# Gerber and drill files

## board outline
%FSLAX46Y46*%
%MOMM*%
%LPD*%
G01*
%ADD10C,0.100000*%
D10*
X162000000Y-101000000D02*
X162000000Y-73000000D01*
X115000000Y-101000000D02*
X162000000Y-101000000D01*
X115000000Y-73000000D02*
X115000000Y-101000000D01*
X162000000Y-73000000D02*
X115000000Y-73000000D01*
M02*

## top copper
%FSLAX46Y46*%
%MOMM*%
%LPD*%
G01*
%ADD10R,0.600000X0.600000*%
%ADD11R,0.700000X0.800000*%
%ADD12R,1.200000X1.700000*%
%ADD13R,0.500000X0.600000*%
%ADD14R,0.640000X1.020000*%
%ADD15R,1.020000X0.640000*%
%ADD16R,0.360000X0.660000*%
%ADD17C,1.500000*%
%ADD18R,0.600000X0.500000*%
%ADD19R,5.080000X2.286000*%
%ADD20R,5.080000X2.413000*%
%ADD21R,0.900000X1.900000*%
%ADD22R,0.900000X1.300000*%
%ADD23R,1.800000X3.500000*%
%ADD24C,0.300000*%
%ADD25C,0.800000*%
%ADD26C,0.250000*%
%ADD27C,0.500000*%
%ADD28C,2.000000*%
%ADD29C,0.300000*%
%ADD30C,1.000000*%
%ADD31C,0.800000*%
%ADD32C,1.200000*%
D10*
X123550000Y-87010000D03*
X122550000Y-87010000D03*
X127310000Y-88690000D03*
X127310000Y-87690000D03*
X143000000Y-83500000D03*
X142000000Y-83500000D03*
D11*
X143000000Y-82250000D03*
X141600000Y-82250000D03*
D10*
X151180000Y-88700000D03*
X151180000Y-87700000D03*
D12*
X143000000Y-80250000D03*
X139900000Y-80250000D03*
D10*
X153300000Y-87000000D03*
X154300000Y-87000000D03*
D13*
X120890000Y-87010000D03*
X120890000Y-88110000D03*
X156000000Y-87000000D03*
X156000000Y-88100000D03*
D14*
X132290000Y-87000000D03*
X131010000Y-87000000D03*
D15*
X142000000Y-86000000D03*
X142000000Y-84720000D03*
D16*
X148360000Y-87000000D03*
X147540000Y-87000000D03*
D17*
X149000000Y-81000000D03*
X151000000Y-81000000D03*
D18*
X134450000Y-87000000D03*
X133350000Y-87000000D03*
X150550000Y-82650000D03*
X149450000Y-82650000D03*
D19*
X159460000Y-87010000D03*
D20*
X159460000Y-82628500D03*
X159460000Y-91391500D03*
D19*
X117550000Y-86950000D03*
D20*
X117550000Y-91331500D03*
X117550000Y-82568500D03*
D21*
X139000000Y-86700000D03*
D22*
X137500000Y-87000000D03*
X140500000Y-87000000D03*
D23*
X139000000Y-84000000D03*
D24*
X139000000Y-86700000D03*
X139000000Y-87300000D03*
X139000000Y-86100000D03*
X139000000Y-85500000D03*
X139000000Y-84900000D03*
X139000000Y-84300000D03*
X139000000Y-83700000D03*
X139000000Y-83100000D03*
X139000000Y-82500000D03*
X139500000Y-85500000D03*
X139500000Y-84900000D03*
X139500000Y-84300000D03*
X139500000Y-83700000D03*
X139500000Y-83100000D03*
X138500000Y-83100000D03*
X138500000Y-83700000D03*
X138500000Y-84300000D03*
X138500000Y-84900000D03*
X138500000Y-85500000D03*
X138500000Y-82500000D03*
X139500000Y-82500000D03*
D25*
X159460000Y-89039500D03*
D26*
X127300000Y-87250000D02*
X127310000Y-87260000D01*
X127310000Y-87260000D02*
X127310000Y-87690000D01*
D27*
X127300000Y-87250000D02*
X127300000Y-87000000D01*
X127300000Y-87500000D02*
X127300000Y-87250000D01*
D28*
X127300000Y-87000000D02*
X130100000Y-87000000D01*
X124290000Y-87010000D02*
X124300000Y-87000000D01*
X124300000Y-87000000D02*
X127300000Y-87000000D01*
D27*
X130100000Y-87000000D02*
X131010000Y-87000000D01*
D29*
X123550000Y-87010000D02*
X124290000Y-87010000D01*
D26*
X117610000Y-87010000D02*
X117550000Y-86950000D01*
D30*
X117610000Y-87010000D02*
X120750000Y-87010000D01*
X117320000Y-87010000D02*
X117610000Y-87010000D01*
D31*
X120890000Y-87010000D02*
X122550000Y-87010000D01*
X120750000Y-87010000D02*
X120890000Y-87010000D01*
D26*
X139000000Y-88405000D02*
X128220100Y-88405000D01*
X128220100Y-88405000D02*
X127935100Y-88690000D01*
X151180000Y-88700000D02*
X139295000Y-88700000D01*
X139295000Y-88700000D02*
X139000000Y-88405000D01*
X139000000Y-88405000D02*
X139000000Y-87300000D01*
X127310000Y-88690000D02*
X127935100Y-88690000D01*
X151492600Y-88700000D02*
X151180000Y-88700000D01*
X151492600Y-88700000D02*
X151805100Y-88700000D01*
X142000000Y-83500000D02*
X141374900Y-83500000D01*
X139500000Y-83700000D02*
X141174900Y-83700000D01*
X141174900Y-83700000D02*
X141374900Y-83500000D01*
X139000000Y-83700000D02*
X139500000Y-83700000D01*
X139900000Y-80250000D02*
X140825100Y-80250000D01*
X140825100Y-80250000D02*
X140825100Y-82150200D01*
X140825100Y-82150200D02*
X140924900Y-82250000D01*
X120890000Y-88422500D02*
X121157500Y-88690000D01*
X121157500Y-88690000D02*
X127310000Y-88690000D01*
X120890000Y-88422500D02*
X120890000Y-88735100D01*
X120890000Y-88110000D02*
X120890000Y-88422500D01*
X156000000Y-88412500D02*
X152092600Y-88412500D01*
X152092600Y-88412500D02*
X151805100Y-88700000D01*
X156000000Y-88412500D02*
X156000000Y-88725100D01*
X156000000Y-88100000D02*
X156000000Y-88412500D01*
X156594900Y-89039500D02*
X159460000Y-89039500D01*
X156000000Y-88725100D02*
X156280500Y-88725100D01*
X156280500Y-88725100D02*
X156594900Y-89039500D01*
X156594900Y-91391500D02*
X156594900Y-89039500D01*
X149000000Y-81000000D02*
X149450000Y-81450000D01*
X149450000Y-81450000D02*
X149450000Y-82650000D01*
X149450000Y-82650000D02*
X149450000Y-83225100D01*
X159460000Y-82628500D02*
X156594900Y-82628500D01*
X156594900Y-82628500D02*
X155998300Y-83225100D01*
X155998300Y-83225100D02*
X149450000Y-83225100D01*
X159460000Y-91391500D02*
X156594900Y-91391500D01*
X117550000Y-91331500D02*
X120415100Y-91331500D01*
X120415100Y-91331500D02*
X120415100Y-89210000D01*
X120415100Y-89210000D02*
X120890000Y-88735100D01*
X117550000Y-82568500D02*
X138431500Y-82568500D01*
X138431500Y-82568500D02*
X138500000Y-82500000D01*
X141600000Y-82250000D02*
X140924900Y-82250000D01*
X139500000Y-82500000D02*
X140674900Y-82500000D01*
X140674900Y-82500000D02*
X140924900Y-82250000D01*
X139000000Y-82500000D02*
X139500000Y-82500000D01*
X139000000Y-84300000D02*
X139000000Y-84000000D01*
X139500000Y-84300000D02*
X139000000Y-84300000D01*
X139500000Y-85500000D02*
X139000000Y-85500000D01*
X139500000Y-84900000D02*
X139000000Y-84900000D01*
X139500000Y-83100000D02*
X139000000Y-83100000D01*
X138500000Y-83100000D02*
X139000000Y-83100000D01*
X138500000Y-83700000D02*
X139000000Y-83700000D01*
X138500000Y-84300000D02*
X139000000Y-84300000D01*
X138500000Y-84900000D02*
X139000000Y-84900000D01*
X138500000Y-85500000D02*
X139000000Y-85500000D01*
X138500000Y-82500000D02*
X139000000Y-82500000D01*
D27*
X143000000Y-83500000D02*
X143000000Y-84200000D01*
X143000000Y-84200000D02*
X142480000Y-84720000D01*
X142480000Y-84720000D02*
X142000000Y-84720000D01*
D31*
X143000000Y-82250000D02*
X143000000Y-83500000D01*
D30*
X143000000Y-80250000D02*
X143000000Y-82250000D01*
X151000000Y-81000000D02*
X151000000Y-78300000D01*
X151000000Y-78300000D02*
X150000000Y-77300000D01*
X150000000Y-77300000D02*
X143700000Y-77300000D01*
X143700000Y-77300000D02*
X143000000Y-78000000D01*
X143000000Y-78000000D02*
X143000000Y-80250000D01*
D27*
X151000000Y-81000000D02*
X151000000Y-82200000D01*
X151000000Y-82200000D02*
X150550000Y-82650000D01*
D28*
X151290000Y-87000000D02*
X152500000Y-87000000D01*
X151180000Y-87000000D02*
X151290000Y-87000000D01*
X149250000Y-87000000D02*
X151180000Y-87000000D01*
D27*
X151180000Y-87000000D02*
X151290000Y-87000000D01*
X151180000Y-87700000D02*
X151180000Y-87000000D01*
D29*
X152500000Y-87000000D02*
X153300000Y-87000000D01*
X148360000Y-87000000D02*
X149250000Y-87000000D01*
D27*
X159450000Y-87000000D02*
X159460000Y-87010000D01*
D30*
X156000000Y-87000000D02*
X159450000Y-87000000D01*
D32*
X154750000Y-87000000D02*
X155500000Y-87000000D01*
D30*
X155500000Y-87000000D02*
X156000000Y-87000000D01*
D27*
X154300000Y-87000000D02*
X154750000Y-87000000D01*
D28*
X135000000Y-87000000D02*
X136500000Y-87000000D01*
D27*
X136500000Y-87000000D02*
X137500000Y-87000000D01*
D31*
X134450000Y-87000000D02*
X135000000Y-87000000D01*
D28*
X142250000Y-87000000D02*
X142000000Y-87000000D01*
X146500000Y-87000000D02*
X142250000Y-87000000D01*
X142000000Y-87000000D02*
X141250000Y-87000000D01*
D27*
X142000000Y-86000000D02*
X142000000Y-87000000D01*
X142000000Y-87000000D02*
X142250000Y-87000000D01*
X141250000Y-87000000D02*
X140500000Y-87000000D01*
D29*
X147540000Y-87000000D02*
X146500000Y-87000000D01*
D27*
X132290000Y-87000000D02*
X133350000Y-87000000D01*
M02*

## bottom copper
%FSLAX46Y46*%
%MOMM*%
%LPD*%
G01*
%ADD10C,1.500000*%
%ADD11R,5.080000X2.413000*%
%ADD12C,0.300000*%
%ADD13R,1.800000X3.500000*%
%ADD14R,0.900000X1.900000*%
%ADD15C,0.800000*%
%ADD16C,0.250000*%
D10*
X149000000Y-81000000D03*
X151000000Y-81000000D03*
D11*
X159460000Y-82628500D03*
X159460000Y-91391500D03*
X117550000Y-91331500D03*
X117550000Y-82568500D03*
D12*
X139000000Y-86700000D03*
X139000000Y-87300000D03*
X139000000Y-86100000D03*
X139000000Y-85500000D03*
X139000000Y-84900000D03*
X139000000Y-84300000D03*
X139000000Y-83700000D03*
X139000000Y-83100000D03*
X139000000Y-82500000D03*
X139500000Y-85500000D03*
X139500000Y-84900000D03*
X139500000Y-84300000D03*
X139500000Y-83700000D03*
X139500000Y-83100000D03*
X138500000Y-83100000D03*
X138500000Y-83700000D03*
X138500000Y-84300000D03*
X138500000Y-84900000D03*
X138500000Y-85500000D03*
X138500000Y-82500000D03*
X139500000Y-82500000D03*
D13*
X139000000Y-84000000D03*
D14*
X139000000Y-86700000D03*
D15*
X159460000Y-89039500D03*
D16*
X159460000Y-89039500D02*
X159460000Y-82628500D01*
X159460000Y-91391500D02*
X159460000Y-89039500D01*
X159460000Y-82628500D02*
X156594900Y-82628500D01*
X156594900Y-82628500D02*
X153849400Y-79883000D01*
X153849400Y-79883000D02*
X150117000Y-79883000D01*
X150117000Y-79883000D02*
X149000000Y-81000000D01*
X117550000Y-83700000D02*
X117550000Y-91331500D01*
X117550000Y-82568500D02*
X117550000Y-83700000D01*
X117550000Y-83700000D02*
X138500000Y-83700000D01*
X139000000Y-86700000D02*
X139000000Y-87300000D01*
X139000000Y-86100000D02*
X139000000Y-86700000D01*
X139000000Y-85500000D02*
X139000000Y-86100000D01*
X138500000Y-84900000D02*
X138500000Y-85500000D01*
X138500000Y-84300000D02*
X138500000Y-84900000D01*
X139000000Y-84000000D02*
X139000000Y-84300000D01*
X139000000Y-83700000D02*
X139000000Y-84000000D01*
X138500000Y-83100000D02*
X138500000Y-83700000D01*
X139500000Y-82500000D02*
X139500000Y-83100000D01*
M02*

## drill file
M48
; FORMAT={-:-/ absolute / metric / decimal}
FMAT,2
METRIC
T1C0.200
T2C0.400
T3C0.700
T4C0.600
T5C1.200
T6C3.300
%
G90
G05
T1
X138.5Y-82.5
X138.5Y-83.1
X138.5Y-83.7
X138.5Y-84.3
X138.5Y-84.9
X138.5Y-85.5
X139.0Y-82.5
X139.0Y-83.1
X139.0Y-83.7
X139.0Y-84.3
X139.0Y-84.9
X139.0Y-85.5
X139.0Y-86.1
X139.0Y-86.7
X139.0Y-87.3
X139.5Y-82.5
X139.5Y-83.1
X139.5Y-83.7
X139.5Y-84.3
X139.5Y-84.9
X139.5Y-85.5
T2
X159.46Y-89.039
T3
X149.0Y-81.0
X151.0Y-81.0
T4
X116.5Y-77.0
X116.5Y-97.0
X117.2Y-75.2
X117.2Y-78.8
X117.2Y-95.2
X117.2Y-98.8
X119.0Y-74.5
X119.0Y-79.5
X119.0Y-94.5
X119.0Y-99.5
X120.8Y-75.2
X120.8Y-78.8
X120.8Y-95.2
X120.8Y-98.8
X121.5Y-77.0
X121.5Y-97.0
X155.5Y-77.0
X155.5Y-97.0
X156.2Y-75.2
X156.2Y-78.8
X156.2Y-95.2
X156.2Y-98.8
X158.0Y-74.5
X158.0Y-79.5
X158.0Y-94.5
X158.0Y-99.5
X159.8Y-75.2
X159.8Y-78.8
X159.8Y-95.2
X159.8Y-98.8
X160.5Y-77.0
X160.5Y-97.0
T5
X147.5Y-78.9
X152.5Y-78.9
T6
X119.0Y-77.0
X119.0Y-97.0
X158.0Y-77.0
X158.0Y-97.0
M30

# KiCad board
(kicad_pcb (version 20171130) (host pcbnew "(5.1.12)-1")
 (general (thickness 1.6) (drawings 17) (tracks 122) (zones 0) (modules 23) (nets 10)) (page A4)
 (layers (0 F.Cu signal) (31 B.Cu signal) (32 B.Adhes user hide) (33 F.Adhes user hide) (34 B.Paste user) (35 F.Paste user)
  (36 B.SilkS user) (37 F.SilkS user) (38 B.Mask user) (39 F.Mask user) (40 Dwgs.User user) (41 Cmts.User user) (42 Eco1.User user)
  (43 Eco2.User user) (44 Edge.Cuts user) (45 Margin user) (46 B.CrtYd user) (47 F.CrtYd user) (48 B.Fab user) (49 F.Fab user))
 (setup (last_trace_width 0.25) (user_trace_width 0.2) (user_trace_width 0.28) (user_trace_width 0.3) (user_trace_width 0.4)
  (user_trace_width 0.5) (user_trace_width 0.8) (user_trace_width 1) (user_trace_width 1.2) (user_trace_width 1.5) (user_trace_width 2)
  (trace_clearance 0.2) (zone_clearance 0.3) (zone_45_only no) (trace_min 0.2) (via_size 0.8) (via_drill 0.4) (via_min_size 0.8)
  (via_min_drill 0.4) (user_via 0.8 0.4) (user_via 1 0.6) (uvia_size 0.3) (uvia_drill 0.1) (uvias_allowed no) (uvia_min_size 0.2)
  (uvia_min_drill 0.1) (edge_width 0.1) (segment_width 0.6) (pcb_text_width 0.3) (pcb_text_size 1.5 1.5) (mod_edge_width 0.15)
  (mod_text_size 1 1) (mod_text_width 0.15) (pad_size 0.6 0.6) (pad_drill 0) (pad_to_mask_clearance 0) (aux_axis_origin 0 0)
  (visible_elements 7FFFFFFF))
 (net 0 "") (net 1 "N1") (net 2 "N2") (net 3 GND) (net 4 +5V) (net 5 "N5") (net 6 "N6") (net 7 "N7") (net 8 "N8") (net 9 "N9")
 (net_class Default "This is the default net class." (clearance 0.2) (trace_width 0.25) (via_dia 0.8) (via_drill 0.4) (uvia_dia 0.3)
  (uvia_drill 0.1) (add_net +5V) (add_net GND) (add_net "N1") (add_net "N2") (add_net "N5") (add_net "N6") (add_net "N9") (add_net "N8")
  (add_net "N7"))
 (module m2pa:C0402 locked (layer F.Cu) (at 123.55 87.01 180)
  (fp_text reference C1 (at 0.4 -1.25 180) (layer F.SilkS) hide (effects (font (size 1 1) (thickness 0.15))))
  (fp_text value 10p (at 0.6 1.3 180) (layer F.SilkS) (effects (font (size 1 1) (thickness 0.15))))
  (pad 1 smd rect (at 0 0 180) (size 0.6 0.6) (layers F.Cu F.Paste F.Mask) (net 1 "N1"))
  (pad 2 smd rect (at 1 0 180) (size 0.6 0.6) (layers F.Cu F.Paste F.Mask) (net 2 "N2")))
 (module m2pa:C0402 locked (layer F.Cu) (at 127.31 88.69 90)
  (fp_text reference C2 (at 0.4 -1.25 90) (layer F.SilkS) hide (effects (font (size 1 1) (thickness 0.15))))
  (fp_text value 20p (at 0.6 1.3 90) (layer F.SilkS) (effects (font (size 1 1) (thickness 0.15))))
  (pad 1 smd rect (at 0 0 90) (size 0.6 0.6) (layers F.Cu F.Paste F.Mask) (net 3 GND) (zone_connect 2))
  (pad 2 smd rect (at 1 0 90) (size 0.6 0.6) (layers F.Cu F.Paste F.Mask) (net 1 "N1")))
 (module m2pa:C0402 (layer F.Cu) (at 143 83.5 180)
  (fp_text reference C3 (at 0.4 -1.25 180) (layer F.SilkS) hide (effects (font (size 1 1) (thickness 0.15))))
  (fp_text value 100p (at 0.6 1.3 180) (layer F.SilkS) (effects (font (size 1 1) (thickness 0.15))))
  (pad 1 smd rect (at 0 0 180) (size 0.6 0.6) (layers F.Cu F.Paste F.Mask) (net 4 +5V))
  (pad 2 smd rect (at 1 0 180) (size 0.6 0.6) (layers F.Cu F.Paste F.Mask) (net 3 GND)))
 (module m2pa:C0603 (layer F.Cu) (at 143 82.25 180)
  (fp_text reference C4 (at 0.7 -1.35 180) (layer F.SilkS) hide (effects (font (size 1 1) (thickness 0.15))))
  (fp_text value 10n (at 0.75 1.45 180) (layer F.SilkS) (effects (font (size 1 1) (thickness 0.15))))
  (pad 1 smd rect (at 0 0 180) (size 0.7 0.8) (layers F.Cu F.Paste F.Mask) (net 4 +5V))
  (pad 2 smd rect (at 1.4 0 180) (size 0.7 0.8) (layers F.Cu F.Paste F.Mask) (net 3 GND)))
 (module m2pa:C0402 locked (layer F.Cu) (at 151.18 88.7 90)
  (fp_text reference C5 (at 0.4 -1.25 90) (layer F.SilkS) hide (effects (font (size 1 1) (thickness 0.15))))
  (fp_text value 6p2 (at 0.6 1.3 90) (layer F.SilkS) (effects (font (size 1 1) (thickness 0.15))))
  (pad 1 smd rect (at 0 0 90) (size 0.6 0.6) (layers F.Cu F.Paste F.Mask) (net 3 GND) (zone_connect 2))
  (pad 2 smd rect (at 1 0 90) (size 0.6 0.6) (layers F.Cu F.Paste F.Mask) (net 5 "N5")))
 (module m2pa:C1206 (layer F.Cu) (at 143 80.25 180)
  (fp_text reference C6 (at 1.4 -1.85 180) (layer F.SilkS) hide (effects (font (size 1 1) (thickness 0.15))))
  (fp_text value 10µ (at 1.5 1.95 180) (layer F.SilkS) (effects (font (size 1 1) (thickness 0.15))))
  (pad 1 smd rect (at 0 0 180) (size 1.2 1.7) (layers F.Cu F.Paste F.Mask) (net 4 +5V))
  (pad 2 smd rect (at 3.1 0 180) (size 1.2 1.7) (layers F.Cu F.Paste F.Mask) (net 3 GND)))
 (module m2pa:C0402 (layer F.Cu) (at 153.3 87)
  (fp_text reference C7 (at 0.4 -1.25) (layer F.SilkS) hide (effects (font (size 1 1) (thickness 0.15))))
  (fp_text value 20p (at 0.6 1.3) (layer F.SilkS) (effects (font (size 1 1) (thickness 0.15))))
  (pad 1 smd rect (at 0 0) (size 0.6 0.6) (layers F.Cu F.Paste F.Mask) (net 5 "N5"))
  (pad 2 smd rect (at 1 0) (size 0.6 0.6) (layers F.Cu F.Paste F.Mask) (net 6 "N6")))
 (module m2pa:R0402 (layer F.Cu) (at 120.89 87.01 270)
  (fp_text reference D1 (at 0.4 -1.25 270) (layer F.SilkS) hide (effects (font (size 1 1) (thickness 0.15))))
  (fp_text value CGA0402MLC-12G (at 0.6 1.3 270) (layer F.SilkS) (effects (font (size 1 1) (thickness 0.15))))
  (pad 1 smd rect (at 0 0 270) (size 0.6 0.5) (layers F.Cu F.Paste F.Mask) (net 2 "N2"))
  (pad 2 smd rect (at 1.1 0 270) (size 0.6 0.5) (layers F.Cu F.Paste F.Mask) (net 3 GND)))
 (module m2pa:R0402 (layer F.Cu) (at 156 87 270)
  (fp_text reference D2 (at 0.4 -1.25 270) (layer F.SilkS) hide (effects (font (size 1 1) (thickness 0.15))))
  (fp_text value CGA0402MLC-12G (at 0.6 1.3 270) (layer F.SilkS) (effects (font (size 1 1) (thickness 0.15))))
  (pad 1 smd rect (at 0 0 270) (size 0.6 0.5) (layers F.Cu F.Paste F.Mask) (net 6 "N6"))
  (pad 2 smd rect (at 1.1 0 270) (size 0.6 0.5) (layers F.Cu F.Paste F.Mask) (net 3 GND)))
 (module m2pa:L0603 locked (layer F.Cu) (at 132.29 87 180)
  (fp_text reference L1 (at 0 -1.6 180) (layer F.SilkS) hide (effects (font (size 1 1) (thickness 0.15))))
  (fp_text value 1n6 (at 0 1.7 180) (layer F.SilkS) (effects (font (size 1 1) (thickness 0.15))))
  (pad 1 smd rect (at 0 0 180) (size 0.64 1.02) (layers F.Cu F.Paste F.Mask) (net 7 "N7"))
  (pad 2 smd rect (at 1.28 0 180) (size 0.64 1.02) (layers F.Cu F.Paste F.Mask) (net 1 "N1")))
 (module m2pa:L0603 (layer F.Cu) (at 142 86 90)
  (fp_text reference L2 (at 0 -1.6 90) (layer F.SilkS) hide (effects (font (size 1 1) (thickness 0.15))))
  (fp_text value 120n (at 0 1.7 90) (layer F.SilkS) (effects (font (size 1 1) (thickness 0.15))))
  (pad 1 smd rect (at 0 0 90) (size 0.64 1.02) (layers F.Cu F.Paste F.Mask) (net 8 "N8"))
  (pad 2 smd rect (at 1.28 0 90) (size 0.64 1.02) (layers F.Cu F.Paste F.Mask) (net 4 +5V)))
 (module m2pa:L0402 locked (layer F.Cu) (at 148.36 87 180)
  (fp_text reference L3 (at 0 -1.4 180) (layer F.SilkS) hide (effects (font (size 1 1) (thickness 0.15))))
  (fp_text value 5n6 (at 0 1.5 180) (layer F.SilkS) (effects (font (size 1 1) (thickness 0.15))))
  (pad 1 smd rect (at 0 0 180) (size 0.36 0.66) (layers F.Cu F.Paste F.Mask) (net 5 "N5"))
  (pad 2 smd rect (at 0.82 0 180) (size 0.36 0.66) (layers F.Cu F.Paste F.Mask) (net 8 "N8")))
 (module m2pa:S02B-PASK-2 (layer F.Cu) (at 149 81)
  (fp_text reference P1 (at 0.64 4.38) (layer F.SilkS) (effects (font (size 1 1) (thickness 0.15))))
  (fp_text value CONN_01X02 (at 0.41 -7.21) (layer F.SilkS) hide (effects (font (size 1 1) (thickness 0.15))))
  (pad 1 thru_hole circle (at 0 0) (size 1.5 1.5) (drill 0.7) (layers *.Cu *.Mask F.SilkS) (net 3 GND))
  (pad 2 thru_hole circle (at 2 0) (size 1.5 1.5) (drill 0.7) (layers *.Cu *.Mask F.SilkS) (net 4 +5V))
  (pad "" np_thru_hole circle (at -1.5 -2.1) (size 1.2 1.2) (drill 1.2) (layers *.Cu *.Mask F.SilkS))
  (pad "" np_thru_hole circle (at 3.5 -2.1) (size 1.2 1.2) (drill 1.2) (layers *.Cu *.Mask F.SilkS)))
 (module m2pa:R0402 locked (layer F.Cu) (at 134.45 87 180)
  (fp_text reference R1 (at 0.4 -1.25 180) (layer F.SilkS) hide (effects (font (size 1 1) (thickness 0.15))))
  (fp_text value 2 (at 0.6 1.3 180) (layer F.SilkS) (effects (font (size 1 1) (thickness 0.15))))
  (pad 1 smd rect (at 0 0 180) (size 0.6 0.5) (layers F.Cu F.Paste F.Mask) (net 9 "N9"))
  (pad 2 smd rect (at 1.1 0 180) (size 0.6 0.5) (layers F.Cu F.Paste F.Mask) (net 7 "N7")))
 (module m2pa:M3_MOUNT (layer F.Cu) (at 158 77)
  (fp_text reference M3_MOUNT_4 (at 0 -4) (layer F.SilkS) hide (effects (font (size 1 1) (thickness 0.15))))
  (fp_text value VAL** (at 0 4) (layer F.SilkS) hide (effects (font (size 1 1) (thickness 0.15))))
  (pad "" np_thru_hole circle (at 0 0) (size 3.3 3.3) (drill 3.3) (layers *.Cu *.Mask F.Paste F.SilkS) (solder_mask_margin 1.5)
   (clearance 1.65))
  (pad "" np_thru_hole circle (at 0 -2.5) (size 0.6 0.6) (drill 0.6) (layers *.Cu *.Mask F.SilkS))
  (pad "" np_thru_hole circle (at 2.5 0) (size 0.6 0.6) (drill 0.6) (layers *.Cu *.Mask F.SilkS))
  (pad "" np_thru_hole circle (at 0 2.5) (size 0.6 0.6) (drill 0.6) (layers *.Cu *.Mask F.SilkS))
  (pad "" np_thru_hole circle (at -2.5 0) (size 0.6 0.6) (drill 0.6) (layers *.Cu *.Mask F.SilkS))
  (pad "" np_thru_hole circle (at -1.8 -1.8) (size 0.6 0.6) (drill 0.6) (layers *.Cu *.Mask F.SilkS))
  (pad "" np_thru_hole circle (at 1.8 -1.8) (size 0.6 0.6) (drill 0.6) (layers *.Cu *.Mask F.SilkS))
  (pad "" np_thru_hole circle (at -1.8 1.8) (size 0.6 0.6) (drill 0.6) (layers *.Cu *.Mask F.SilkS))
  (pad "" np_thru_hole circle (at 1.8 1.8) (size 0.6 0.6) (drill 0.6) (layers *.Cu *.Mask F.SilkS)))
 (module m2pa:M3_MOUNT (layer F.Cu) (at 119 97)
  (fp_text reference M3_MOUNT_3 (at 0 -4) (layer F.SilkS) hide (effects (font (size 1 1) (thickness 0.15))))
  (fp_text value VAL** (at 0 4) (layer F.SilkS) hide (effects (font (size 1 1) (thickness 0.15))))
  (pad "" np_thru_hole circle (at 0 0) (size 3.3 3.3) (drill 3.3) (layers *.Cu *.Mask F.Paste F.SilkS) (solder_mask_margin 1.5)
   (clearance 1.65))
  (pad "" np_thru_hole circle (at 0 -2.5) (size 0.6 0.6) (drill 0.6) (layers *.Cu *.Mask F.SilkS))
  (pad "" np_thru_hole circle (at 2.5 0) (size 0.6 0.6) (drill 0.6) (layers *.Cu *.Mask F.SilkS))
  (pad "" np_thru_hole circle (at 0 2.5) (size 0.6 0.6) (drill 0.6) (layers *.Cu *.Mask F.SilkS))
  (pad "" np_thru_hole circle (at -2.5 0) (size 0.6 0.6) (drill 0.6) (layers *.Cu *.Mask F.SilkS))
  (pad "" np_thru_hole circle (at -1.8 -1.8) (size 0.6 0.6) (drill 0.6) (layers *.Cu *.Mask F.SilkS))
  (pad "" np_thru_hole circle (at 1.8 -1.8) (size 0.6 0.6) (drill 0.6) (layers *.Cu *.Mask F.SilkS))
  (pad "" np_thru_hole circle (at -1.8 1.8) (size 0.6 0.6) (drill 0.6) (layers *.Cu *.Mask F.SilkS))
  (pad "" np_thru_hole circle (at 1.8 1.8) (size 0.6 0.6) (drill 0.6) (layers *.Cu *.Mask F.SilkS)))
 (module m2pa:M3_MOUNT (layer F.Cu) (at 158 97)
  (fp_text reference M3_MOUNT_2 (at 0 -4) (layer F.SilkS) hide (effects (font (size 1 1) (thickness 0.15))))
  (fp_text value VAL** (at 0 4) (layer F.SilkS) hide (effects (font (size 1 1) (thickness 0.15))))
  (pad "" np_thru_hole circle (at 0 0) (size 3.3 3.3) (drill 3.3) (layers *.Cu *.Mask F.Paste F.SilkS) (solder_mask_margin 1.5)
   (clearance 1.65))
  (pad "" np_thru_hole circle (at 0 -2.5) (size 0.6 0.6) (drill 0.6) (layers *.Cu *.Mask F.SilkS))
  (pad "" np_thru_hole circle (at 2.5 0) (size 0.6 0.6) (drill 0.6) (layers *.Cu *.Mask F.SilkS))
  (pad "" np_thru_hole circle (at 0 2.5) (size 0.6 0.6) (drill 0.6) (layers *.Cu *.Mask F.SilkS))
  (pad "" np_thru_hole circle (at -2.5 0) (size 0.6 0.6) (drill 0.6) (layers *.Cu *.Mask F.SilkS))
  (pad "" np_thru_hole circle (at -1.8 -1.8) (size 0.6 0.6) (drill 0.6) (layers *.Cu *.Mask F.SilkS))
  (pad "" np_thru_hole circle (at 1.8 -1.8) (size 0.6 0.6) (drill 0.6) (layers *.Cu *.Mask F.SilkS))
  (pad "" np_thru_hole circle (at -1.8 1.8) (size 0.6 0.6) (drill 0.6) (layers *.Cu *.Mask F.SilkS))
  (pad "" np_thru_hole circle (at 1.8 1.8) (size 0.6 0.6) (drill 0.6) (layers *.Cu *.Mask F.SilkS)))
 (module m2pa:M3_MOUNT (layer F.Cu) (at 119 77)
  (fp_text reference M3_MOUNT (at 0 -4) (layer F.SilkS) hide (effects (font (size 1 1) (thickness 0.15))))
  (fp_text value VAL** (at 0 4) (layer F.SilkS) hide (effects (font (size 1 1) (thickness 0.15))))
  (pad "" np_thru_hole circle (at 0 0) (size 3.3 3.3) (drill 3.3) (layers *.Cu *.Mask F.Paste F.SilkS) (solder_mask_margin 1.5)
   (clearance 1.65))
  (pad "" np_thru_hole circle (at 0 -2.5) (size 0.6 0.6) (drill 0.6) (layers *.Cu *.Mask F.SilkS))
  (pad "" np_thru_hole circle (at 2.5 0) (size 0.6 0.6) (drill 0.6) (layers *.Cu *.Mask F.SilkS))
  (pad "" np_thru_hole circle (at 0 2.5) (size 0.6 0.6) (drill 0.6) (layers *.Cu *.Mask F.SilkS))
  (pad "" np_thru_hole circle (at -2.5 0) (size 0.6 0.6) (drill 0.6) (layers *.Cu *.Mask F.SilkS))
  (pad "" np_thru_hole circle (at -1.8 -1.8) (size 0.6 0.6) (drill 0.6) (layers *.Cu *.Mask F.SilkS))
  (pad "" np_thru_hole circle (at 1.8 -1.8) (size 0.6 0.6) (drill 0.6) (layers *.Cu *.Mask F.SilkS))
  (pad "" np_thru_hole circle (at -1.8 1.8) (size 0.6 0.6) (drill 0.6) (layers *.Cu *.Mask F.SilkS))
  (pad "" np_thru_hole circle (at 1.8 1.8) (size 0.6 0.6) (drill 0.6) (layers *.Cu *.Mask F.SilkS)))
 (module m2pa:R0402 (layer F.Cu) (at 150.55 82.65 180)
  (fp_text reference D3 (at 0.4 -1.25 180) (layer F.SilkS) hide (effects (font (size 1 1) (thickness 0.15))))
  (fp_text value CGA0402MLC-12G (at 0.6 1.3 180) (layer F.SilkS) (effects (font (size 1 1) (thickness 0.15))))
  (pad 1 smd rect (at 0 0 180) (size 0.6 0.5) (layers F.Cu F.Paste F.Mask) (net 4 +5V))
  (pad 2 smd rect (at 1.1 0 180) (size 0.6 0.5) (layers F.Cu F.Paste F.Mask) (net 3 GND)))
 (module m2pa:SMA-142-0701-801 (layer F.Cu) (at 159.46 87.01 270)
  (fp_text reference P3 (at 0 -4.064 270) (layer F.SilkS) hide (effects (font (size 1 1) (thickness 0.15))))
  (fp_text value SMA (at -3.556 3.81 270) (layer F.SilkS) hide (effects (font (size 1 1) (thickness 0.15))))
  (pad 1 smd rect (at 0 0 270) (size 2.286 5.08) (layers F.Cu F.Mask) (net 6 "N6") (zone_connect 2))
  (pad 2 smd rect (at -4.3815 0 270) (size 2.413 5.08) (layers F.Cu F.Mask) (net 3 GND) (zone_connect 2))
  (pad 3 smd rect (at 4.3815 0 270) (size 2.413 5.08) (layers F.Cu F.Mask) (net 3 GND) (zone_connect 2))
  (pad 4 smd rect (at -4.3815 0 270) (size 2.413 5.08) (layers B.Cu B.Mask) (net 3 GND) (zone_connect 2))
  (pad 5 smd rect (at 4.3815 0 270) (size 2.413 5.08) (layers B.Cu B.Mask) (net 3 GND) (zone_connect 2)))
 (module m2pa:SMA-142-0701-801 (layer F.Cu) (at 117.55 86.95 90)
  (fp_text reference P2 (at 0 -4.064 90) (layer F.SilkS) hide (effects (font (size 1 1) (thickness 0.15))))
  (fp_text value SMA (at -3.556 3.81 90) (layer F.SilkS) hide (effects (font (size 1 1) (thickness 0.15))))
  (pad 1 smd rect (at 0 0 90) (size 2.286 5.08) (layers F.Cu F.Mask) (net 2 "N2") (zone_connect 2))
  (pad 2 smd rect (at -4.3815 0 90) (size 2.413 5.08) (layers F.Cu F.Mask) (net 3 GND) (zone_connect 2))
  (pad 3 smd rect (at 4.3815 0 90) (size 2.413 5.08) (layers F.Cu F.Mask) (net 3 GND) (zone_connect 2))
  (pad 4 smd rect (at -4.3815 0 90) (size 2.413 5.08) (layers B.Cu B.Mask) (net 3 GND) (zone_connect 2))
  (pad 5 smd rect (at 4.3815 0 90) (size 2.413 5.08) (layers B.Cu B.Mask) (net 3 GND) (zone_connect 2)))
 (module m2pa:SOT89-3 (layer F.Cu) (at 139 87)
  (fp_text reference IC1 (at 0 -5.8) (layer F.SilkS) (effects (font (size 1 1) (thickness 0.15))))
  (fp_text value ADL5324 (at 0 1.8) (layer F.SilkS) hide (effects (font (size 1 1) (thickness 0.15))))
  (pad 2 smd rect (at 0 -0.3 180) (size 0.9 1.9) (layers F.Cu F.Paste F.Mask) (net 3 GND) (zone_connect 2))
  (pad 1 smd rect (at -1.5 0 180) (size 0.9 1.3) (layers F.Cu F.Paste F.Mask) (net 9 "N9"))
  (pad 3 smd rect (at 1.5 0 180) (size 0.9 1.3) (layers F.Cu F.Paste F.Mask) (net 8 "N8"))
  (pad 2 smd rect (at 0 -3 180) (size 1.8 3.5) (layers F.Cu F.Paste F.Mask) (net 3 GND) (zone_connect 2))
  (pad 2 thru_hole circle (at 0 -0.3 180) (size 0.3 0.3) (drill 0.2) (layers *.Cu F.SilkS F.Mask) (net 3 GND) (zone_connect 2))
  (pad 2 thru_hole circle (at 0 0.3 180) (size 0.3 0.3) (drill 0.2) (layers *.Cu F.SilkS F.Mask) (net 3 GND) (zone_connect 2))
  (pad 2 thru_hole circle (at 0 -0.9 180) (size 0.3 0.3) (drill 0.2) (layers *.Cu F.SilkS F.Mask) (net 3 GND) (zone_connect 2))
  (pad 2 thru_hole circle (at 0 -1.5 180) (size 0.3 0.3) (drill 0.2) (layers *.Cu F.SilkS F.Mask) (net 3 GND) (zone_connect 2))
  (pad 2 thru_hole circle (at 0 -2.1 180) (size 0.3 0.3) (drill 0.2) (layers *.Cu F.SilkS F.Mask) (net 3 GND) (zone_connect 2))
  (pad 2 thru_hole circle (at 0 -2.7 180) (size 0.3 0.3) (drill 0.2) (layers *.Cu F.SilkS F.Mask) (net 3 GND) (zone_connect 2))
  (pad 2 thru_hole circle (at 0 -3.3 180) (size 0.3 0.3) (drill 0.2) (layers *.Cu F.SilkS F.Mask) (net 3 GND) (zone_connect 2))
  (pad 2 thru_hole circle (at 0 -3.9 180) (size 0.3 0.3) (drill 0.2) (layers *.Cu F.SilkS F.Mask) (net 3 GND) (zone_connect 2))
  (pad 2 thru_hole circle (at 0 -4.5 180) (size 0.3 0.3) (drill 0.2) (layers *.Cu F.SilkS F.Mask) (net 3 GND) (zone_connect 2))
  (pad 2 thru_hole circle (at 0.5 -1.5 180) (size 0.3 0.3) (drill 0.2) (layers *.Cu F.SilkS F.Mask) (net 3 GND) (zone_connect 2))
  (pad 2 thru_hole circle (at 0.5 -2.1 180) (size 0.3 0.3) (drill 0.2) (layers *.Cu F.SilkS F.Mask) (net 3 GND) (zone_connect 2))
  (pad 2 thru_hole circle (at 0.5 -2.7 180) (size 0.3 0.3) (drill 0.2) (layers *.Cu F.SilkS F.Mask) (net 3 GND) (zone_connect 2))
  (pad 2 thru_hole circle (at 0.5 -3.3 180) (size 0.3 0.3) (drill 0.2) (layers *.Cu F.SilkS F.Mask) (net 3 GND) (zone_connect 2))
  (pad 2 thru_hole circle (at 0.5 -3.9 180) (size 0.3 0.3) (drill 0.2) (layers *.Cu F.SilkS F.Mask) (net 3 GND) (zone_connect 2))
  (pad 2 thru_hole circle (at -0.5 -3.9 180) (size 0.3 0.3) (drill 0.2) (layers *.Cu F.SilkS F.Mask) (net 3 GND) (zone_connect 2))
  (pad 2 thru_hole circle (at -0.5 -3.3 180) (size 0.3 0.3) (drill 0.2) (layers *.Cu F.SilkS F.Mask) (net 3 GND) (zone_connect 2))
  (pad 2 thru_hole circle (at -0.5 -2.7 180) (size 0.3 0.3) (drill 0.2) (layers *.Cu F.SilkS F.Mask) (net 3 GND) (zone_connect 2))
  (pad 2 thru_hole circle (at -0.5 -2.1 180) (size 0.3 0.3) (drill 0.2) (layers *.Cu F.SilkS F.Mask) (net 3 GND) (zone_connect 2))
  (pad 2 thru_hole circle (at -0.5 -1.5 180) (size 0.3 0.3) (drill 0.2) (layers *.Cu F.SilkS F.Mask) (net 3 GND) (zone_connect 2))
  (pad 2 thru_hole circle (at -0.5 -4.5 180) (size 0.3 0.3) (drill 0.2) (layers *.Cu F.SilkS F.Mask) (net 3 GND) (zone_connect 2))
  (pad 2 thru_hole circle (at 0.5 -4.5 180) (size 0.3 0.3) (drill 0.2) (layers *.Cu F.SilkS F.Mask) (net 3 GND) (zone_connect 2))
  (pad 2 smd rect (at 0 -3 180) (size 1.8 3.5) (layers B.Cu) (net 3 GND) (zone_connect 2))
  (pad 2 smd rect (at 0 -0.3 180) (size 0.9 1.9) (layers B.Cu) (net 3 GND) (zone_connect 2)))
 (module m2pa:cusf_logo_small (layer F.Cu) (at 124 80)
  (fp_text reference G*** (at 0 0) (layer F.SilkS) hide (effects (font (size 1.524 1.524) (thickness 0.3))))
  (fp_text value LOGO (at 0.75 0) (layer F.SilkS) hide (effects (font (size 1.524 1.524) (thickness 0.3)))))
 (gr_line (start 162 101) (end 162 73) (angle 90) (layer Edge.Cuts) (width 0.1))
 (gr_line (start 115 101) (end 162 101) (angle 90) (layer Edge.Cuts) (width 0.1))
 (gr_line (start 115 73) (end 115 101) (angle 90) (layer Edge.Cuts) (width 0.1))
 (gr_line (start 162 73) (end 115 73) (angle 90) (layer Edge.Cuts) (width 0.1))
 (segment (start 127.3 87.25) (end 127.31 87.26) (width 0.25) (layer F.Cu) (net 1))
 (segment (start 127.31 87.26) (end 127.31 87.69) (width 0.25) (layer F.Cu) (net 1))
 (segment (start 127.3 87.25) (end 127.3 87) (width 0.5) (layer F.Cu) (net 1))
 (segment (start 127.3 87.5) (end 127.3 87.25) (width 0.5) (layer F.Cu) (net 1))
 (segment (start 127.3 87) (end 130.1 87) (width 2) (layer F.Cu) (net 1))
 (segment (start 124.29 87.01) (end 124.3 87) (width 2) (layer F.Cu) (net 1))
 (segment (start 124.3 87) (end 127.3 87) (width 2) (layer F.Cu) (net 1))
 (segment (start 130.1 87) (end 131.01 87) (width 0.5) (layer F.Cu) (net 1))
 (segment (start 123.55 87.01) (end 124.29 87.01) (width 0.3) (layer F.Cu) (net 1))
 (segment (start 117.61 87.01) (end 117.55 86.95) (width 0.25) (layer F.Cu) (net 2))
 (segment (start 117.61 87.01) (end 120.75 87.01) (width 1) (layer F.Cu) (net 2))
 (segment (start 117.32 87.01) (end 117.61 87.01) (width 1) (layer F.Cu) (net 2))
 (segment (start 120.89 87.01) (end 122.55 87.01) (width 0.8) (layer F.Cu) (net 2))
 (segment (start 120.75 87.01) (end 120.89 87.01) (width 0.8) (layer F.Cu) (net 2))
 (segment (start 139 88.405) (end 128.2201 88.405) (width 0.25) (layer F.Cu) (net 3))
 (segment (start 128.2201 88.405) (end 127.9351 88.69) (width 0.25) (layer F.Cu) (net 3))
 (segment (start 151.18 88.7) (end 139.295 88.7) (width 0.25) (layer F.Cu) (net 3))
 (segment (start 139.295 88.7) (end 139 88.405) (width 0.25) (layer F.Cu) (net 3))
 (segment (start 139 88.405) (end 139 87.3) (width 0.25) (layer F.Cu) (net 3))
 (segment (start 127.31 88.69) (end 127.9351 88.69) (width 0.25) (layer F.Cu) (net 3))
 (segment (start 151.4926 88.7) (end 151.18 88.7) (width 0.25) (layer F.Cu) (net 3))
 (segment (start 151.4926 88.7) (end 151.8051 88.7) (width 0.25) (layer F.Cu) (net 3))
 (segment (start 142 83.5) (end 141.3749 83.5) (width 0.25) (layer F.Cu) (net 3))
 (segment (start 139.5 83.7) (end 141.1749 83.7) (width 0.25) (layer F.Cu) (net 3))
 (segment (start 141.1749 83.7) (end 141.3749 83.5) (width 0.25) (layer F.Cu) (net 3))
 (segment (start 139 83.7) (end 139.5 83.7) (width 0.25) (layer F.Cu) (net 3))
 (segment (start 139.9 80.25) (end 140.8251 80.25) (width 0.25) (layer F.Cu) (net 3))
 (segment (start 140.8251 80.25) (end 140.8251 82.1502) (width 0.25) (layer F.Cu) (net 3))
 (segment (start 140.8251 82.1502) (end 140.9249 82.25) (width 0.25) (layer F.Cu) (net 3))
 (segment (start 120.89 88.4225) (end 121.1575 88.69) (width 0.25) (layer F.Cu) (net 3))
 (segment (start 121.1575 88.69) (end 127.31 88.69) (width 0.25) (layer F.Cu) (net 3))
 (segment (start 120.89 88.4225) (end 120.89 88.7351) (width 0.25) (layer F.Cu) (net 3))
 (segment (start 120.89 88.11) (end 120.89 88.4225) (width 0.25) (layer F.Cu) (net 3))
 (segment (start 156 88.4125) (end 152.0926 88.4125) (width 0.25) (layer F.Cu) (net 3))
 (segment (start 152.0926 88.4125) (end 151.8051 88.7) (width 0.25) (layer F.Cu) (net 3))
 (segment (start 156 88.4125) (end 156 88.7251) (width 0.25) (layer F.Cu) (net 3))
 (segment (start 156 88.1) (end 156 88.4125) (width 0.25) (layer F.Cu) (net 3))
 (segment (start 156.5949 89.0395) (end 159.46 89.0395) (width 0.25) (layer F.Cu) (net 3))
 (segment (start 156 88.7251) (end 156.2805 88.7251) (width 0.25) (layer F.Cu) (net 3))
 (segment (start 156.2805 88.7251) (end 156.5949 89.0395) (width 0.25) (layer F.Cu) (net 3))
 (segment (start 156.5949 91.3915) (end 156.5949 89.0395) (width 0.25) (layer F.Cu) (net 3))
 (segment (start 159.46 89.0395) (end 159.46 82.6285) (width 0.25) (layer B.Cu) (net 3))
 (segment (start 159.46 91.3915) (end 159.46 89.0395) (width 0.25) (layer B.Cu) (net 3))
 (segment (start 149 81) (end 149.45 81.45) (width 0.25) (layer F.Cu) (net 3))
 (segment (start 149.45 81.45) (end 149.45 82.65) (width 0.25) (layer F.Cu) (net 3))
 (segment (start 149.45 82.65) (end 149.45 83.2251) (width 0.25) (layer F.Cu) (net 3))
 (segment (start 159.46 82.6285) (end 156.5949 82.6285) (width 0.25) (layer F.Cu) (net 3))
 (segment (start 156.5949 82.6285) (end 155.9983 83.2251) (width 0.25) (layer F.Cu) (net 3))
 (segment (start 155.9983 83.2251) (end 149.45 83.2251) (width 0.25) (layer F.Cu) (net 3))
 (segment (start 159.46 91.3915) (end 156.5949 91.3915) (width 0.25) (layer F.Cu) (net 3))
 (segment (start 159.46 82.6285) (end 156.5949 82.6285) (width 0.25) (layer B.Cu) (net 3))
 (segment (start 156.5949 82.6285) (end 153.8494 79.883) (width 0.25) (layer B.Cu) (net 3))
 (segment (start 153.8494 79.883) (end 150.117 79.883) (width 0.25) (layer B.Cu) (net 3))
 (segment (start 150.117 79.883) (end 149 81) (width 0.25) (layer B.Cu) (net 3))
 (segment (start 117.55 91.3315) (end 120.4151 91.3315) (width 0.25) (layer F.Cu) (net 3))
 (segment (start 120.4151 91.3315) (end 120.4151 89.21) (width 0.25) (layer F.Cu) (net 3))
 (segment (start 120.4151 89.21) (end 120.89 88.7351) (width 0.25) (layer F.Cu) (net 3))
 (segment (start 117.55 82.5685) (end 138.4315 82.5685) (width 0.25) (layer F.Cu) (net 3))
 (segment (start 138.4315 82.5685) (end 138.5 82.5) (width 0.25) (layer F.Cu) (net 3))
 (segment (start 117.55 83.7) (end 117.55 91.3315) (width 0.25) (layer B.Cu) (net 3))
 (segment (start 117.55 82.5685) (end 117.55 83.7) (width 0.25) (layer B.Cu) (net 3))
 (segment (start 117.55 83.7) (end 138.5 83.7) (width 0.25) (layer B.Cu) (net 3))
 (segment (start 141.6 82.25) (end 140.9249 82.25) (width 0.25) (layer F.Cu) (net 3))
 (segment (start 139.5 82.5) (end 140.6749 82.5) (width 0.25) (layer F.Cu) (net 3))
 (segment (start 140.6749 82.5) (end 140.9249 82.25) (width 0.25) (layer F.Cu) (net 3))
 (segment (start 139 82.5) (end 139.5 82.5) (width 0.25) (layer F.Cu) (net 3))
 (segment (start 139 84.3) (end 139 84) (width 0.25) (layer F.Cu) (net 3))
 (segment (start 139.5 84.3) (end 139 84.3) (width 0.25) (layer F.Cu) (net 3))
 (segment (start 139 86.7) (end 139 87.3) (width 0.25) (layer B.Cu) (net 3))
 (segment (start 139 86.1) (end 139 86.7) (width 0.25) (layer B.Cu) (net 3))
 (segment (start 139 85.5) (end 139 86.1) (width 0.25) (layer B.Cu) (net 3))
 (segment (start 138.5 84.9) (end 138.5 85.5) (width 0.25) (layer B.Cu) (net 3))
 (segment (start 138.5 84.3) (end 138.5 84.9) (width 0.25) (layer B.Cu) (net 3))
 (segment (start 139 84) (end 139 84.3) (width 0.25) (layer B.Cu) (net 3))
 (segment (start 139 83.7) (end 139 84) (width 0.25) (layer B.Cu) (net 3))
 (segment (start 138.5 83.1) (end 138.5 83.7) (width 0.25) (layer B.Cu) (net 3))
 (segment (start 139.5 82.5) (end 139.5 83.1) (width 0.25) (layer B.Cu) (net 3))
 (segment (start 139.5 85.5) (end 139 85.5) (width 0.25) (layer F.Cu) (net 3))
 (segment (start 139.5 84.9) (end 139 84.9) (width 0.25) (layer F.Cu) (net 3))
 (segment (start 139.5 83.1) (end 139 83.1) (width 0.25) (layer F.Cu) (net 3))
 (segment (start 138.5 83.1) (end 139 83.1) (width 0.25) (layer F.Cu) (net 3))
 (segment (start 138.5 83.7) (end 139 83.7) (width 0.25) (layer F.Cu) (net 3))
 (segment (start 138.5 84.3) (end 139 84.3) (width 0.25) (layer F.Cu) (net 3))
 (segment (start 138.5 84.9) (end 139 84.9) (width 0.25) (layer F.Cu) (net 3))
 (segment (start 138.5 85.5) (end 139 85.5) (width 0.25) (layer F.Cu) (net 3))
 (segment (start 138.5 82.5) (end 139 82.5) (width 0.25) (layer F.Cu) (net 3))
 (via (at 159.46 89.0395) (size 0.8) (layers F.Cu B.Cu) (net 3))
 (segment (start 143 83.5) (end 143 84.2) (width 0.5) (layer F.Cu) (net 4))
 (segment (start 143 84.2) (end 142.48 84.72) (width 0.5) (layer F.Cu) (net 4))
 (segment (start 142.48 84.72) (end 142 84.72) (width 0.5) (layer F.Cu) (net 4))
 (segment (start 143 82.25) (end 143 83.5) (width 0.8) (layer F.Cu) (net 4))
 (segment (start 143 80.25) (end 143 82.25) (width 1) (layer F.Cu) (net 4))
 (segment (start 151 81) (end 151 78.3) (width 1) (layer F.Cu) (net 4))
 (segment (start 151 78.3) (end 150 77.3) (width 1) (layer F.Cu) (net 4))
 (segment (start 150 77.3) (end 143.7 77.3) (width 1) (layer F.Cu) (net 4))
 (segment (start 143.7 77.3) (end 143 78) (width 1) (layer F.Cu) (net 4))
 (segment (start 143 78) (end 143 80.25) (width 1) (layer F.Cu) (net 4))
 (segment (start 151 81) (end 151 82.2) (width 0.5) (layer F.Cu) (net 4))
 (segment (start 151 82.2) (end 150.55 82.65) (width 0.5) (layer F.Cu) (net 4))
 (segment (start 151.29 87) (end 152.5 87) (width 2) (layer F.Cu) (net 5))
 (segment (start 151.18 87) (end 151.29 87) (width 2) (layer F.Cu) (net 5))
 (segment (start 149.25 87) (end 151.18 87) (width 2) (layer F.Cu) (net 5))
 (segment (start 151.18 87) (end 151.29 87) (width 0.5) (layer F.Cu) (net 5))
 (segment (start 151.18 87.7) (end 151.18 87) (width 0.5) (layer F.Cu) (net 5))
 (segment (start 152.5 87) (end 153.3 87) (width 0.3) (layer F.Cu) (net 5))
 (segment (start 148.36 87) (end 149.25 87) (width 0.3) (layer F.Cu) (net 5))
 (segment (start 159.45 87) (end 159.46 87.01) (width 0.5) (layer F.Cu) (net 6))
 (segment (start 156 87) (end 159.45 87) (width 1) (layer F.Cu) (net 6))
 (segment (start 154.75 87) (end 155.5 87) (width 1.2) (layer F.Cu) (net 6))
 (segment (start 155.5 87) (end 156 87) (width 1) (layer F.Cu) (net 6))
 (segment (start 154.3 87) (end 154.75 87) (width 0.5) (layer F.Cu) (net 6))
 (segment (start 135 87) (end 136.5 87) (width 2) (layer F.Cu) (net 9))
 (segment (start 136.5 87) (end 137.5 87) (width 0.5) (layer F.Cu) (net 9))
 (segment (start 134.45 87) (end 135 87) (width 0.8) (layer F.Cu) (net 9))
 (segment (start 142.25 87) (end 142 87) (width 2) (layer F.Cu) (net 8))
 (segment (start 146.5 87) (end 142.25 87) (width 2) (layer F.Cu) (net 8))
 (segment (start 142 87) (end 141.25 87) (width 2) (layer F.Cu) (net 8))
 (segment (start 142 86) (end 142 87) (width 0.5) (layer F.Cu) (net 8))
 (segment (start 142 87) (end 142.25 87) (width 0.5) (layer F.Cu) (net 8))
 (segment (start 141.25 87) (end 140.5 87) (width 0.5) (layer F.Cu) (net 8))
 (segment (start 147.54 87) (end 146.5 87) (width 0.3) (layer F.Cu) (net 8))
 (segment (start 132.29 87) (end 133.35 87) (width 0.5) (layer F.Cu) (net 7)))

